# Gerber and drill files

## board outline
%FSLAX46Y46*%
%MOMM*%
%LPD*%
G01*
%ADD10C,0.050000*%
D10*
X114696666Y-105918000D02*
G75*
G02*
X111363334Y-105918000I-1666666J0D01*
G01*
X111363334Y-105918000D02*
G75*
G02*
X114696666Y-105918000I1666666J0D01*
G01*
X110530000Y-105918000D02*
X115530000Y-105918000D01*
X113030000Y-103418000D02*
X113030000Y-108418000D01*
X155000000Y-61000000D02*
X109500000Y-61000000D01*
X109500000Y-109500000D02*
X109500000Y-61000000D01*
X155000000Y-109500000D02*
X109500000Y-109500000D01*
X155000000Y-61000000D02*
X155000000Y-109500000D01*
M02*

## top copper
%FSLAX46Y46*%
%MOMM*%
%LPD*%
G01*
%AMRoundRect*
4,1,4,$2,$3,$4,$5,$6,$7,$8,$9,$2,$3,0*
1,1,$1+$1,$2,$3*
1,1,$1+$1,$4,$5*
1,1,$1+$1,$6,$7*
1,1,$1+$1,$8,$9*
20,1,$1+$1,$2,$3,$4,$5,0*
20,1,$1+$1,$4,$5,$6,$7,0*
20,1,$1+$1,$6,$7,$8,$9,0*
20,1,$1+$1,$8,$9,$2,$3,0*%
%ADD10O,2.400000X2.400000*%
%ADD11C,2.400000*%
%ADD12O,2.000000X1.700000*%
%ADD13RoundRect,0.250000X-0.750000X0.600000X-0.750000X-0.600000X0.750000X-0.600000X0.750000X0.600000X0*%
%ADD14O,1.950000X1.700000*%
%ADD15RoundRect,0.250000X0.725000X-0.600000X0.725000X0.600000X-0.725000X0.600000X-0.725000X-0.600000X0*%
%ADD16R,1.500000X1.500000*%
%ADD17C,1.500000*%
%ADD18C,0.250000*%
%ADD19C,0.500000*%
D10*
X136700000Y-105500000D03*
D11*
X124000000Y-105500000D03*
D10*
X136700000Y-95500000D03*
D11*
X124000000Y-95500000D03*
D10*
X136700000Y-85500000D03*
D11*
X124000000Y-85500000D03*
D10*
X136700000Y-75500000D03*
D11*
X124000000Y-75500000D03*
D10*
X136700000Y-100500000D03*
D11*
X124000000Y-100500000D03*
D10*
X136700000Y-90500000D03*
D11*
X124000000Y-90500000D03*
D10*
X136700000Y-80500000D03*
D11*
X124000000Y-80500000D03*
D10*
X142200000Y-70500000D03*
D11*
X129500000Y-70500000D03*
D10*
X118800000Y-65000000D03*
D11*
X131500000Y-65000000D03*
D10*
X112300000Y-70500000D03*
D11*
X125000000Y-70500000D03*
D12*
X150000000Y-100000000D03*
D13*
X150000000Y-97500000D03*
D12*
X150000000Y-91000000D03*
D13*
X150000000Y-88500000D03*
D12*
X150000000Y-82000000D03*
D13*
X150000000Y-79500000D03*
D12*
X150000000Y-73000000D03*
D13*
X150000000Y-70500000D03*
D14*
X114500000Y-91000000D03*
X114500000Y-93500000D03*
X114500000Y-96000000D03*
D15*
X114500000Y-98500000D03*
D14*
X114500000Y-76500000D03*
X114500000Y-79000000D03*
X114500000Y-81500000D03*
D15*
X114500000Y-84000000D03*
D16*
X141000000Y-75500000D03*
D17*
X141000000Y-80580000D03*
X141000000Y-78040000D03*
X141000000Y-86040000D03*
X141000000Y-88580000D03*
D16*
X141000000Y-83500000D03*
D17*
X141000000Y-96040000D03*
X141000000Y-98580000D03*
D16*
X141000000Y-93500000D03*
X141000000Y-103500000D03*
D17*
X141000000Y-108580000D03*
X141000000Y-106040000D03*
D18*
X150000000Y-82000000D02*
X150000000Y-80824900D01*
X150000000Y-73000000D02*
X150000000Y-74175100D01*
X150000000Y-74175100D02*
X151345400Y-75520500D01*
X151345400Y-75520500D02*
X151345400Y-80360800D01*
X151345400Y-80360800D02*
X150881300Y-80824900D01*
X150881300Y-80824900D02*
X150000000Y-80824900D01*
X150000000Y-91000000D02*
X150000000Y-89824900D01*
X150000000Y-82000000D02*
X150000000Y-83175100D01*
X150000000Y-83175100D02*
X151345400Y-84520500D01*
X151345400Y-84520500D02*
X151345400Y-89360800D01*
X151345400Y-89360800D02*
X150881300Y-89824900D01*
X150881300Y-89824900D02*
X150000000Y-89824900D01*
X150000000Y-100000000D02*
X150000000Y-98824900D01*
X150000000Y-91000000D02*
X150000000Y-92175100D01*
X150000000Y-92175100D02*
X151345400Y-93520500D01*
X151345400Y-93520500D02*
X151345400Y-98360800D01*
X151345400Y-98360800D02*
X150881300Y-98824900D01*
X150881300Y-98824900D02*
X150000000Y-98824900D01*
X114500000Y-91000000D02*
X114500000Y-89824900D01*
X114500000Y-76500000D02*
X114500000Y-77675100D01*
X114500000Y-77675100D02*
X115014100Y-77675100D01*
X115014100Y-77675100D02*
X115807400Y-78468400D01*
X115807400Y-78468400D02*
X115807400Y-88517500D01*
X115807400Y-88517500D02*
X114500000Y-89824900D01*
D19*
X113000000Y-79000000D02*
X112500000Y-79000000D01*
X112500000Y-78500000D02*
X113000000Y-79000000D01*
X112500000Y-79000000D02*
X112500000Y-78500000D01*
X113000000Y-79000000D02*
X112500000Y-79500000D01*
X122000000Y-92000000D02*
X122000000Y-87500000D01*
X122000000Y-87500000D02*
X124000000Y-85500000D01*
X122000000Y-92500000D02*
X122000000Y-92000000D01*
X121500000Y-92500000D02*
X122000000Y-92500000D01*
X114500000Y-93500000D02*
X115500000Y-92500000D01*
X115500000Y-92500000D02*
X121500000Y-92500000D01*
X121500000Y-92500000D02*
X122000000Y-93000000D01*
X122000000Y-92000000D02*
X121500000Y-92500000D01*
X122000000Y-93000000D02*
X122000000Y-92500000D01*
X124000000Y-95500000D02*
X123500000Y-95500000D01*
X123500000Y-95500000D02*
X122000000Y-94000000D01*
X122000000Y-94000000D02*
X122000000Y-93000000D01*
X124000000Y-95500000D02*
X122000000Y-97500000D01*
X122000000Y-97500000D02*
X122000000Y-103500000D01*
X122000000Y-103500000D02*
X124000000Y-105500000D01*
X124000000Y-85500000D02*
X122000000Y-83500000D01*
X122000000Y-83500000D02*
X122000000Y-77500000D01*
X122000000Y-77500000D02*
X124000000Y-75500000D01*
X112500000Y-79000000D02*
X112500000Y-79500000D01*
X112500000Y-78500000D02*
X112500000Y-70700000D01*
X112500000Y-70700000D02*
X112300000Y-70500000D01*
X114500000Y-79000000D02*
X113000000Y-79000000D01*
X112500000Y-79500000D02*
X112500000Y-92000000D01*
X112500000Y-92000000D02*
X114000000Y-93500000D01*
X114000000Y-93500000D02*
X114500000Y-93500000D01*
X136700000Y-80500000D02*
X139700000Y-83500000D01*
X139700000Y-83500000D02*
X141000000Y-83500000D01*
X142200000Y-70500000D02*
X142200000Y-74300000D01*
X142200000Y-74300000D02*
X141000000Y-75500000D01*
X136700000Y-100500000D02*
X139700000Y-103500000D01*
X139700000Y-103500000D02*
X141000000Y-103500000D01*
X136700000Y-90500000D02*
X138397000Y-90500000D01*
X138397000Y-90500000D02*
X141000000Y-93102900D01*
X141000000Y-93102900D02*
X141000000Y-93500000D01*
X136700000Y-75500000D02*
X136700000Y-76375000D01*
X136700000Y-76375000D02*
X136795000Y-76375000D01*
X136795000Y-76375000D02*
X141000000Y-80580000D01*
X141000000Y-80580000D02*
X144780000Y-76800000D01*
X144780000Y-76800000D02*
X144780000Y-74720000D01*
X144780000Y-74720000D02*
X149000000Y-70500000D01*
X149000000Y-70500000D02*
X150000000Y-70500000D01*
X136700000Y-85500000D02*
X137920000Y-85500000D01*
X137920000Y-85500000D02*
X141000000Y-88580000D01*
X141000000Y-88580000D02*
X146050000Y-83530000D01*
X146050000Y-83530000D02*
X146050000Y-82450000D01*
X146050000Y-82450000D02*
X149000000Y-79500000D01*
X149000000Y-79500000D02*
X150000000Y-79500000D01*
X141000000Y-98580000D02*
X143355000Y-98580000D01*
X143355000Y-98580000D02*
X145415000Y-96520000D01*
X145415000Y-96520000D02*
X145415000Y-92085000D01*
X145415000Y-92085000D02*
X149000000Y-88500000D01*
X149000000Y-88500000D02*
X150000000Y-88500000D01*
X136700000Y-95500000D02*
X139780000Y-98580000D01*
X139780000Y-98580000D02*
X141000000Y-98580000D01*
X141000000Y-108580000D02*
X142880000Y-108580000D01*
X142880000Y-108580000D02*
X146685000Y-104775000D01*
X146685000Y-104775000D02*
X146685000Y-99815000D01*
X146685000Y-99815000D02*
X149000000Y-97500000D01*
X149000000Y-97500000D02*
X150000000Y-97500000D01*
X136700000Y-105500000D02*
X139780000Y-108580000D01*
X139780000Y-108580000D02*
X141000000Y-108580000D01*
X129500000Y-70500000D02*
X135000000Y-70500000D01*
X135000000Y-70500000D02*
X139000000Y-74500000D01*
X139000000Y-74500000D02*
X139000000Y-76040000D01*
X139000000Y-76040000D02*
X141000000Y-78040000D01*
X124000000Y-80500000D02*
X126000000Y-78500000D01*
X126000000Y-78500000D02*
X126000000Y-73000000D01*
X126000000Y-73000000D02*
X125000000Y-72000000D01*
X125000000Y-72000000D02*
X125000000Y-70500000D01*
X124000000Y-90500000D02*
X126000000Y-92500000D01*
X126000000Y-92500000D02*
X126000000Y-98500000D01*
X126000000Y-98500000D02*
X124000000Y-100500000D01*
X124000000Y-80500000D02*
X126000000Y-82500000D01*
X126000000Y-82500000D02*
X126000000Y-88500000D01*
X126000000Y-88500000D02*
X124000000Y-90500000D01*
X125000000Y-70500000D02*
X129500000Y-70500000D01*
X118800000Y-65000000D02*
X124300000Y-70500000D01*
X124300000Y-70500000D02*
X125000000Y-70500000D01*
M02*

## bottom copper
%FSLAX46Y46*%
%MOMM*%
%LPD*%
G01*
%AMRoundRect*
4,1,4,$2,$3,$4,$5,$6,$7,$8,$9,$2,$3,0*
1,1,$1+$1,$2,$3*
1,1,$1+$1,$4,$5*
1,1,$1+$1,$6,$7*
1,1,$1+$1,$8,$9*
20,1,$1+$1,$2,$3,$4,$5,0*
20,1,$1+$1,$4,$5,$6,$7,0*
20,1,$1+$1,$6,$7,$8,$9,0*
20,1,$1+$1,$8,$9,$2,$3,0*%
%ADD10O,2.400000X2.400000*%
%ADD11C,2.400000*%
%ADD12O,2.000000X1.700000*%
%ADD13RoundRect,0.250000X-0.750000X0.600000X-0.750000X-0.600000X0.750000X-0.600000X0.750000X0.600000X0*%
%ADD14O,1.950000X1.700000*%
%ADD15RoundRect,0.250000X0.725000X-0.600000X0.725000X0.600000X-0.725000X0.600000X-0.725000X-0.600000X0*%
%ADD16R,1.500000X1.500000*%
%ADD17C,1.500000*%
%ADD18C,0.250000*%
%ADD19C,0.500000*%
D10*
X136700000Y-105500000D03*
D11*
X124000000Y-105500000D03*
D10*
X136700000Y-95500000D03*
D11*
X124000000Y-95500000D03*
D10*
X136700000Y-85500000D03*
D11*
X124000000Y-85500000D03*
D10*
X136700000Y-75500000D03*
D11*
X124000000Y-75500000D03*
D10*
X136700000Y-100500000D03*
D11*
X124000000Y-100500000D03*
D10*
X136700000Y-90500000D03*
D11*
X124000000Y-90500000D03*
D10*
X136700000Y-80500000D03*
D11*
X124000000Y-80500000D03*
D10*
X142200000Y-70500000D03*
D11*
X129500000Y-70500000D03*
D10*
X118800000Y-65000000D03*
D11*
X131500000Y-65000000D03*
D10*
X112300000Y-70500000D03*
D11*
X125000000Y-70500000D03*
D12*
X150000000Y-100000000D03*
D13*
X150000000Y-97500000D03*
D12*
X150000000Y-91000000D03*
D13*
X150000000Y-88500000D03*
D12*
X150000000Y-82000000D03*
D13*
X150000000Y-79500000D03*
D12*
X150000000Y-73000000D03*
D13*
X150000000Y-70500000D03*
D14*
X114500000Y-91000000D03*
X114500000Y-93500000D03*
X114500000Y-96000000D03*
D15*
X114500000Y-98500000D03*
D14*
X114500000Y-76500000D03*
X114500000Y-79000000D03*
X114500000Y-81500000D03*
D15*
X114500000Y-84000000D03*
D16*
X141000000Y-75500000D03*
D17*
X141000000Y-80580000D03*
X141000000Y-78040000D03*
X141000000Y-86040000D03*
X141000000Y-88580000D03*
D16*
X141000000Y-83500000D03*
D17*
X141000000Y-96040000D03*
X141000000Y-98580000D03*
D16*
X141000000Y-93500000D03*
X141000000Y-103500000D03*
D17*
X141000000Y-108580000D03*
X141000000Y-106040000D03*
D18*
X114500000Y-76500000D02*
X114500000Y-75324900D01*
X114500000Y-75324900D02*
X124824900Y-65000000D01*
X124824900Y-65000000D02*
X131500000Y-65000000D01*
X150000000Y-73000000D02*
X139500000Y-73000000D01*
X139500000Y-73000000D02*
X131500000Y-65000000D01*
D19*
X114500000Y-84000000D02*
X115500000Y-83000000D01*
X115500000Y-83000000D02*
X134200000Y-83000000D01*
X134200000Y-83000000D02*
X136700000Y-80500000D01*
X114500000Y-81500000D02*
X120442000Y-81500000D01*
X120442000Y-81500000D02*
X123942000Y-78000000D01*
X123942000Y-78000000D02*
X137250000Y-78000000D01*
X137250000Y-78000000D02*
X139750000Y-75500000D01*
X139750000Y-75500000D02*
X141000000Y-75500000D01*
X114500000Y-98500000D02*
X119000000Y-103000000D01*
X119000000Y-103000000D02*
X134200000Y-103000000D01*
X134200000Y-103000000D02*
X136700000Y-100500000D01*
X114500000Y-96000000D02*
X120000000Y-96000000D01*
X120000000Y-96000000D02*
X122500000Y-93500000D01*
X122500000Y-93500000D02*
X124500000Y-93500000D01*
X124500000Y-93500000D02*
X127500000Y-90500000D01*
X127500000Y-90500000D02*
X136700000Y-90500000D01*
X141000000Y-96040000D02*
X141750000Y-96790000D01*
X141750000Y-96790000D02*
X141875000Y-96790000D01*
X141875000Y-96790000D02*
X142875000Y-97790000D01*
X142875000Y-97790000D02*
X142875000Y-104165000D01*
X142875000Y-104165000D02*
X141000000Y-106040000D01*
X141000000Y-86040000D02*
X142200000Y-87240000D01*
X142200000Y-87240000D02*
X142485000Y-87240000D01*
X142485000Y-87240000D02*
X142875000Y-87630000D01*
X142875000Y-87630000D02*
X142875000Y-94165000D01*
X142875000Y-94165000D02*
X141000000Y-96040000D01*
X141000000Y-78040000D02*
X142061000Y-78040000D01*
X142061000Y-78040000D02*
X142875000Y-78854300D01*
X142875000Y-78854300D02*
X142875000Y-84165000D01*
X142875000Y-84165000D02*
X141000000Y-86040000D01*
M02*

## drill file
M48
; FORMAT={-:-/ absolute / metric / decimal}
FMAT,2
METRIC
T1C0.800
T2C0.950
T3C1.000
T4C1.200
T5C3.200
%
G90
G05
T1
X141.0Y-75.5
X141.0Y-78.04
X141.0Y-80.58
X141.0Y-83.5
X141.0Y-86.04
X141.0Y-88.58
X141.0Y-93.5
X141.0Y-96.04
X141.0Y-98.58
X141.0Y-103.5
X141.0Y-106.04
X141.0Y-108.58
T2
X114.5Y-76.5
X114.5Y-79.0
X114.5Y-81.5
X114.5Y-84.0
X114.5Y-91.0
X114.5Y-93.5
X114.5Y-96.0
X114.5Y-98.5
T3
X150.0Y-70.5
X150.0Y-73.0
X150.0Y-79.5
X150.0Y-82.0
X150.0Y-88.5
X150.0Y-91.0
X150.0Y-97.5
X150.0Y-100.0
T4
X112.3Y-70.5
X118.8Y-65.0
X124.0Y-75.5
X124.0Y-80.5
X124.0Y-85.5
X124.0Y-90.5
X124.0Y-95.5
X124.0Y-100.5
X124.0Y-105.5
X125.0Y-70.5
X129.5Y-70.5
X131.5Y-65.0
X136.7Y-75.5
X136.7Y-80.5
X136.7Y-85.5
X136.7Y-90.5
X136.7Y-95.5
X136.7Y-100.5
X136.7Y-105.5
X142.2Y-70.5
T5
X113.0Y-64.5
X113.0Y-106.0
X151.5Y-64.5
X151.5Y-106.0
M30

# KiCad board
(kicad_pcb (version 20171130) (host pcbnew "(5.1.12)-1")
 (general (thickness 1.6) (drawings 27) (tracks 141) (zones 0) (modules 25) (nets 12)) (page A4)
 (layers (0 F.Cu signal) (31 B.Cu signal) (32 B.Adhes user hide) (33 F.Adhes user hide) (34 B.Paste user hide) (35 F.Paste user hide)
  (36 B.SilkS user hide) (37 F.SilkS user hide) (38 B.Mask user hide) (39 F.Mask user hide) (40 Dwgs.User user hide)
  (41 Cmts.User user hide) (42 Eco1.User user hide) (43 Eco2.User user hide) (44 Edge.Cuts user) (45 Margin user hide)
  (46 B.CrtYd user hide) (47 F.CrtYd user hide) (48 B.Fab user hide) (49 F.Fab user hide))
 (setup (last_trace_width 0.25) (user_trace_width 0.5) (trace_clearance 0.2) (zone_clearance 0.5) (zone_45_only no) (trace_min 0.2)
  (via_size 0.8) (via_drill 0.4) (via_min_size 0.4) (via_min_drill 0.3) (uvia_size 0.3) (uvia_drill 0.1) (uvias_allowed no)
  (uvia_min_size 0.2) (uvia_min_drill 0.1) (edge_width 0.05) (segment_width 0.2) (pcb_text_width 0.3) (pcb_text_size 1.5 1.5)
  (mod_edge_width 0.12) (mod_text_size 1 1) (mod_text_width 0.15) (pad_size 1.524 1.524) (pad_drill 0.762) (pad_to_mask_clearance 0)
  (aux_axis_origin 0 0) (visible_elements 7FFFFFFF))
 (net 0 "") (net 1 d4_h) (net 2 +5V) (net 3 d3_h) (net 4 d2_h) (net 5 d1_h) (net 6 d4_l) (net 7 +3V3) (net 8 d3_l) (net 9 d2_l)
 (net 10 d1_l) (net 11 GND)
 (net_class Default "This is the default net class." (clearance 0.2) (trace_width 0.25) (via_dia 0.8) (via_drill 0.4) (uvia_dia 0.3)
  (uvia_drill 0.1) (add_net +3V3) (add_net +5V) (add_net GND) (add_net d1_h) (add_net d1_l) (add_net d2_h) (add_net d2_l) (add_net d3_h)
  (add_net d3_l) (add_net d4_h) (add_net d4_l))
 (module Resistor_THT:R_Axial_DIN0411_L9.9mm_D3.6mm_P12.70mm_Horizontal (layer F.Cu) (at 124 105.5)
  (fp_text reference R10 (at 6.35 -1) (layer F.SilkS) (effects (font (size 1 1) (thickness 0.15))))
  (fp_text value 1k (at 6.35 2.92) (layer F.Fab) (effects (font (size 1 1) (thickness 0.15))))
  (pad 2 thru_hole oval (at 12.7 0) (size 2.4 2.4) (drill 1.2) (layers *.Cu *.Mask) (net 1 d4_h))
  (pad 1 thru_hole circle (at 0 0) (size 2.4 2.4) (drill 1.2) (layers *.Cu *.Mask) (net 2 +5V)))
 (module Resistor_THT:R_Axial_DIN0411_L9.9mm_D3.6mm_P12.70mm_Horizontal (layer F.Cu) (at 124 95.5)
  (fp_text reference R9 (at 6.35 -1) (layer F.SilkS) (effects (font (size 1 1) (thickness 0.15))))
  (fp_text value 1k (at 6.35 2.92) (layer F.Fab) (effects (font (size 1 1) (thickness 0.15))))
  (pad 2 thru_hole oval (at 12.7 0) (size 2.4 2.4) (drill 1.2) (layers *.Cu *.Mask) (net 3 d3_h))
  (pad 1 thru_hole circle (at 0 0) (size 2.4 2.4) (drill 1.2) (layers *.Cu *.Mask) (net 2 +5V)))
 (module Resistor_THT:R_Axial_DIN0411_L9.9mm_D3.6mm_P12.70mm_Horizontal (layer F.Cu) (at 124 85.5)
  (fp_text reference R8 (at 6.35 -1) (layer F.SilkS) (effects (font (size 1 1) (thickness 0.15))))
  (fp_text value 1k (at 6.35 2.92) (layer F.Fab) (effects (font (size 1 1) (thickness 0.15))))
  (pad 2 thru_hole oval (at 12.7 0) (size 2.4 2.4) (drill 1.2) (layers *.Cu *.Mask) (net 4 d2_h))
  (pad 1 thru_hole circle (at 0 0) (size 2.4 2.4) (drill 1.2) (layers *.Cu *.Mask) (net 2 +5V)))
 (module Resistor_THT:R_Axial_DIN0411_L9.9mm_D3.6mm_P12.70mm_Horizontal (layer F.Cu) (at 124 75.5)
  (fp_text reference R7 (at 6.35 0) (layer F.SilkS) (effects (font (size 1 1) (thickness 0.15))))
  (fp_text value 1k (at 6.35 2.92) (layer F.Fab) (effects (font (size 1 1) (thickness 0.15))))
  (pad 2 thru_hole oval (at 12.7 0) (size 2.4 2.4) (drill 1.2) (layers *.Cu *.Mask) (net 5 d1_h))
  (pad 1 thru_hole circle (at 0 0) (size 2.4 2.4) (drill 1.2) (layers *.Cu *.Mask) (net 2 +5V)))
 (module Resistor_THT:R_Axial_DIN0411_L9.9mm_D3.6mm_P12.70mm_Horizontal (layer F.Cu) (at 124 100.5)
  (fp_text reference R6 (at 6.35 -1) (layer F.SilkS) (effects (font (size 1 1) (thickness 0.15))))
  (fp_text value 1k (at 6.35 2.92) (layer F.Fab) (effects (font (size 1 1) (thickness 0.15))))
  (pad 2 thru_hole oval (at 12.7 0) (size 2.4 2.4) (drill 1.2) (layers *.Cu *.Mask) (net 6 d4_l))
  (pad 1 thru_hole circle (at 0 0) (size 2.4 2.4) (drill 1.2) (layers *.Cu *.Mask) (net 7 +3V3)))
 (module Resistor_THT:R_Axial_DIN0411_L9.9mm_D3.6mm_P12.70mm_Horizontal (layer F.Cu) (at 124 90.5)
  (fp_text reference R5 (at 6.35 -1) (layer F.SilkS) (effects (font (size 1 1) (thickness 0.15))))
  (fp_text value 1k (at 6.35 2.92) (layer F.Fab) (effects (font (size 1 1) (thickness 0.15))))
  (pad 2 thru_hole oval (at 12.7 0) (size 2.4 2.4) (drill 1.2) (layers *.Cu *.Mask) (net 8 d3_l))
  (pad 1 thru_hole circle (at 0 0) (size 2.4 2.4) (drill 1.2) (layers *.Cu *.Mask) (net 7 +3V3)))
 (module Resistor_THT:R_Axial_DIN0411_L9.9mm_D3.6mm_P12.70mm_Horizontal (layer F.Cu) (at 124 80.5)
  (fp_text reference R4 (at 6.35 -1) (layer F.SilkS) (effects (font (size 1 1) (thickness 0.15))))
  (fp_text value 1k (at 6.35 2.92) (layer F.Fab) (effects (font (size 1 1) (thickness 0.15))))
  (pad 2 thru_hole oval (at 12.7 0) (size 2.4 2.4) (drill 1.2) (layers *.Cu *.Mask) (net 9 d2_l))
  (pad 1 thru_hole circle (at 0 0) (size 2.4 2.4) (drill 1.2) (layers *.Cu *.Mask) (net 7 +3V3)))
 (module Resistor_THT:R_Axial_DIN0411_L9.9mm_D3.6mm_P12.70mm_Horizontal (layer F.Cu) (at 129.5 70.5)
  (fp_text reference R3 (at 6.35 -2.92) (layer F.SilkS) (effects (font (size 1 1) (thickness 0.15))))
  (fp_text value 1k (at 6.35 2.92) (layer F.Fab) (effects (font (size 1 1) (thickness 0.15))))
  (pad 2 thru_hole oval (at 12.7 0) (size 2.4 2.4) (drill 1.2) (layers *.Cu *.Mask) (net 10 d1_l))
  (pad 1 thru_hole circle (at 0 0) (size 2.4 2.4) (drill 1.2) (layers *.Cu *.Mask) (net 7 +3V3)))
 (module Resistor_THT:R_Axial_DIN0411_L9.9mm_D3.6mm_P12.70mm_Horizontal (layer F.Cu) (at 131.5 65 180)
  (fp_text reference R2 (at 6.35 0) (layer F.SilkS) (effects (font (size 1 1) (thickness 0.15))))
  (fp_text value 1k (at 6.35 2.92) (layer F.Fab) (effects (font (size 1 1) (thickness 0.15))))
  (pad 2 thru_hole oval (at 12.7 0 180) (size 2.4 2.4) (drill 1.2) (layers *.Cu *.Mask) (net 7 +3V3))
  (pad 1 thru_hole circle (at 0 0 180) (size 2.4 2.4) (drill 1.2) (layers *.Cu *.Mask) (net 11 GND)))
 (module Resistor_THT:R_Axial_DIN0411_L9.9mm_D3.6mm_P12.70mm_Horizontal (layer F.Cu) (at 125 70.5 180)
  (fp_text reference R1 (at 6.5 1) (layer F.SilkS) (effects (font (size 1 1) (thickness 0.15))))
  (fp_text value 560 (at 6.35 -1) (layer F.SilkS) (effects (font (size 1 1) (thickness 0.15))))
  (pad 2 thru_hole oval (at 12.7 0 180) (size 2.4 2.4) (drill 1.2) (layers *.Cu *.Mask) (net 2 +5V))
  (pad 1 thru_hole circle (at 0 0 180) (size 2.4 2.4) (drill 1.2) (layers *.Cu *.Mask) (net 7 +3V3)))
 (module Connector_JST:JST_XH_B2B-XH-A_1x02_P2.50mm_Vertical (layer F.Cu) (at 150 97.5 270)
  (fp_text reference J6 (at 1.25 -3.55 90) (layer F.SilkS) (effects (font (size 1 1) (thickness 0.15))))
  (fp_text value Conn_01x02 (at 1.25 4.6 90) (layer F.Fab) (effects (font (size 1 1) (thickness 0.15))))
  (pad 2 thru_hole oval (at 2.5 0 270) (size 1.7 2) (drill 1) (layers *.Cu *.Mask) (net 11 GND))
  (pad 1 thru_hole roundrect (at 0 0 270) (size 1.7 2) (drill 1) (layers *.Cu *.Mask) (roundrect_rratio 0.1470588235294118) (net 1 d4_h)))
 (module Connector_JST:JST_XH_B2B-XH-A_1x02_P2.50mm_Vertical (layer F.Cu) (at 150 88.5 270)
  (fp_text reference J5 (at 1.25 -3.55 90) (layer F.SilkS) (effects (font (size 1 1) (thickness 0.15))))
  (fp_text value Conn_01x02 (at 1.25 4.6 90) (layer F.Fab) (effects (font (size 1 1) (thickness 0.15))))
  (pad 2 thru_hole oval (at 2.5 0 270) (size 1.7 2) (drill 1) (layers *.Cu *.Mask) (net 11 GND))
  (pad 1 thru_hole roundrect (at 0 0 270) (size 1.7 2) (drill 1) (layers *.Cu *.Mask) (roundrect_rratio 0.1470588235294118) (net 3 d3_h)))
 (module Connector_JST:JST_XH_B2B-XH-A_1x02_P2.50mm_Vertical (layer F.Cu) (at 150 79.5 270)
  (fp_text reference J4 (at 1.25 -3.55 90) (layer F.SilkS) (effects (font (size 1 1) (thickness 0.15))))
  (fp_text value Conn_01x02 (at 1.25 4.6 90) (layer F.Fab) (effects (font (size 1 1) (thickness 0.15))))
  (pad 2 thru_hole oval (at 2.5 0 270) (size 1.7 2) (drill 1) (layers *.Cu *.Mask) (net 11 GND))
  (pad 1 thru_hole roundrect (at 0 0 270) (size 1.7 2) (drill 1) (layers *.Cu *.Mask) (roundrect_rratio 0.1470588235294118) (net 4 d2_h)))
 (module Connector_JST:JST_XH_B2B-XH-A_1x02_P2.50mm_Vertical (layer F.Cu) (at 150 70.5 270)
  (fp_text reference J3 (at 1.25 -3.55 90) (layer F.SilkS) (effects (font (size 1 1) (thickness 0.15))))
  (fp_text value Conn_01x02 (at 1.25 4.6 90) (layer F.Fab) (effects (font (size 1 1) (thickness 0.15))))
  (pad 2 thru_hole oval (at 2.5 0 270) (size 1.7 2) (drill 1) (layers *.Cu *.Mask) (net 11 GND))
  (pad 1 thru_hole roundrect (at 0 0 270) (size 1.7 2) (drill 1) (layers *.Cu *.Mask) (roundrect_rratio 0.1470588235294118) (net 5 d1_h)))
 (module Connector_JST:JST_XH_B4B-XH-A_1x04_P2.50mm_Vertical (layer F.Cu) (at 114.5 98.5 90)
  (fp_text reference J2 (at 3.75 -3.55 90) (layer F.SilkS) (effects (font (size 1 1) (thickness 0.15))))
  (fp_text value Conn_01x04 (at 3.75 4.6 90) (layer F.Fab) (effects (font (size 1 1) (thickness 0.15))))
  (pad 4 thru_hole oval (at 7.5 0 90) (size 1.7 1.95) (drill 0.95) (layers *.Cu *.Mask) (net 11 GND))
  (pad 3 thru_hole oval (at 5 0 90) (size 1.7 1.95) (drill 0.95) (layers *.Cu *.Mask) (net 2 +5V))
  (pad 2 thru_hole oval (at 2.5 0 90) (size 1.7 1.95) (drill 0.95) (layers *.Cu *.Mask) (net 8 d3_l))
  (pad 1 thru_hole roundrect (at 0 0 90) (size 1.7 1.95) (drill 0.95) (layers *.Cu *.Mask) (roundrect_rratio 0.1470588235294118)
   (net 6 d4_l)))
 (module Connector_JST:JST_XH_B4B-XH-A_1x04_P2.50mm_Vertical (layer F.Cu) (at 114.5 84 90)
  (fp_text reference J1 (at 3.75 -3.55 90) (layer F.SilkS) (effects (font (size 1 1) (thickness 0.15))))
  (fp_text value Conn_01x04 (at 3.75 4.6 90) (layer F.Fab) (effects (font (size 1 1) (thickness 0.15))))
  (pad 4 thru_hole oval (at 7.5 0 90) (size 1.7 1.95) (drill 0.95) (layers *.Cu *.Mask) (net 11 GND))
  (pad 3 thru_hole oval (at 5 0 90) (size 1.7 1.95) (drill 0.95) (layers *.Cu *.Mask) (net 2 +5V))
  (pad 2 thru_hole oval (at 2.5 0 90) (size 1.7 1.95) (drill 0.95) (layers *.Cu *.Mask) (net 10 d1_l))
  (pad 1 thru_hole roundrect (at 0 0 90) (size 1.7 1.95) (drill 0.95) (layers *.Cu *.Mask) (roundrect_rratio 0.1470588235294118)
   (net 9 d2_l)))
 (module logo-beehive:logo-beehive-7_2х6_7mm (layer F.Cu) (at 140 65)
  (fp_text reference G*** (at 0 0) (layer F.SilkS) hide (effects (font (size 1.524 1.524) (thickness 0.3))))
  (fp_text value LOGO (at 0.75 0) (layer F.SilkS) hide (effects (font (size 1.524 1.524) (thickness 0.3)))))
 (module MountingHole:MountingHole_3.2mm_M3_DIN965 (layer F.Cu) (at 113 106)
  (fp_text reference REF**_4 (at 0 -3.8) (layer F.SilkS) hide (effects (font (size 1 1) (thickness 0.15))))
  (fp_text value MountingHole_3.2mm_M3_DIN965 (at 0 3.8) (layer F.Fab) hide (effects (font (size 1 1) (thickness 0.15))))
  (pad 1 np_thru_hole circle (at 0 0) (size 3.2 3.2) (drill 3.2) (layers *.Cu *.Mask)))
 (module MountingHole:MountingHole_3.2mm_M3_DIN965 (layer F.Cu) (at 151.5 64.5)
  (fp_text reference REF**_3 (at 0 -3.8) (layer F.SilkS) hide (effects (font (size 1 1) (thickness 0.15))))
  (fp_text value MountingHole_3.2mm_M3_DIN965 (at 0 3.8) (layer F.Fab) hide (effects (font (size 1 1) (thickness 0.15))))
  (pad 1 np_thru_hole circle (at 0 0) (size 3.2 3.2) (drill 3.2) (layers *.Cu *.Mask)))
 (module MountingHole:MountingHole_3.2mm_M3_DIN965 (layer F.Cu) (at 113 64.5)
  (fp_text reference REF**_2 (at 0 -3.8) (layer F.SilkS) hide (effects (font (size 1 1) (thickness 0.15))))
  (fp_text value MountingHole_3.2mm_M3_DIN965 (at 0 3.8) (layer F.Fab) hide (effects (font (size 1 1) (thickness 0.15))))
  (pad 1 np_thru_hole circle (at 0 0) (size 3.2 3.2) (drill 3.2) (layers *.Cu *.Mask)))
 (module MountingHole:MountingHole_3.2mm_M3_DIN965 (layer F.Cu) (at 151.5 106)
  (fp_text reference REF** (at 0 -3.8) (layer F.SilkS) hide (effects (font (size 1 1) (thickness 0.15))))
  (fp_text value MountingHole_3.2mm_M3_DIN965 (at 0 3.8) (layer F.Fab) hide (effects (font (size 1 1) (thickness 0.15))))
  (pad 1 np_thru_hole circle (at 0 0) (size 3.2 3.2) (drill 3.2) (layers *.Cu *.Mask)))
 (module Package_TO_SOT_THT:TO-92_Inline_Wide (layer F.Cu) (at 141 75.5 270)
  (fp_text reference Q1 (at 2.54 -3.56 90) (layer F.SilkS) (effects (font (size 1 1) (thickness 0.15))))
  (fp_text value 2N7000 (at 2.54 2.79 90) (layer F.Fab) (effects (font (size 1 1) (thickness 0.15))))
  (pad 1 thru_hole rect (at 0 0) (size 1.5 1.5) (drill 0.8) (layers *.Cu *.Mask) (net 10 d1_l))
  (pad 3 thru_hole circle (at 5.08 0) (size 1.5 1.5) (drill 0.8) (layers *.Cu *.Mask) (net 5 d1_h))
  (pad 2 thru_hole circle (at 2.54 0) (size 1.5 1.5) (drill 0.8) (layers *.Cu *.Mask) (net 7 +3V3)))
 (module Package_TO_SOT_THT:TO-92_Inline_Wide (layer F.Cu) (at 141 83.5 270)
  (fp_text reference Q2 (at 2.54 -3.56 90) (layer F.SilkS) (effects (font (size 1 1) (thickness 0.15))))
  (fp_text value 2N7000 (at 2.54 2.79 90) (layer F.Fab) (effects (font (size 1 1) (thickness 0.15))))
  (pad 2 thru_hole circle (at 2.54 0) (size 1.5 1.5) (drill 0.8) (layers *.Cu *.Mask) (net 7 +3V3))
  (pad 3 thru_hole circle (at 5.08 0) (size 1.5 1.5) (drill 0.8) (layers *.Cu *.Mask) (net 4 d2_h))
  (pad 1 thru_hole rect (at 0 0) (size 1.5 1.5) (drill 0.8) (layers *.Cu *.Mask) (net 9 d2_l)))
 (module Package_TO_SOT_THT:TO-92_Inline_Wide (layer F.Cu) (at 141 93.5 270)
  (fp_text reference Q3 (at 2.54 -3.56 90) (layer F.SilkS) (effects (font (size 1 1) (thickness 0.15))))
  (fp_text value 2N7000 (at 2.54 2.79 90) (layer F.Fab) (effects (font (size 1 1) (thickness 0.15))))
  (pad 2 thru_hole circle (at 2.54 0) (size 1.5 1.5) (drill 0.8) (layers *.Cu *.Mask) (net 7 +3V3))
  (pad 3 thru_hole circle (at 5.08 0) (size 1.5 1.5) (drill 0.8) (layers *.Cu *.Mask) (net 3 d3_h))
  (pad 1 thru_hole rect (at 0 0) (size 1.5 1.5) (drill 0.8) (layers *.Cu *.Mask) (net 8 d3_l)))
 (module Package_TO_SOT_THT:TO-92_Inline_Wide (layer F.Cu) (at 141 103.5 270)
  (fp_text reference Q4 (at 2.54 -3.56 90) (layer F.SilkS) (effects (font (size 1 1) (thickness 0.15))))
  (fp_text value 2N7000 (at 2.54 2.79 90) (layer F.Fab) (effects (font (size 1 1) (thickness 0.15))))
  (pad 1 thru_hole rect (at 0 0) (size 1.5 1.5) (drill 0.8) (layers *.Cu *.Mask) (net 6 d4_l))
  (pad 3 thru_hole circle (at 5.08 0) (size 1.5 1.5) (drill 0.8) (layers *.Cu *.Mask) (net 1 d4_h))
  (pad 2 thru_hole circle (at 2.54 0) (size 1.5 1.5) (drill 0.8) (layers *.Cu *.Mask) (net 7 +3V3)))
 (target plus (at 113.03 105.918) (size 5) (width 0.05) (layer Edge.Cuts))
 (gr_line (start 155 61) (end 109.5 61) (layer Edge.Cuts) (width 0.05))
 (gr_line (start 109.5 109.5) (end 109.5 61) (layer Edge.Cuts) (width 0.05))
 (gr_line (start 155 109.5) (end 109.5 109.5) (layer Edge.Cuts) (width 0.05))
 (gr_line (start 155 61) (end 155 109.5) (layer Edge.Cuts) (width 0.05))
 (segment (start 150 82) (end 150 80.8249) (width 0.25) (layer F.Cu) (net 11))
 (segment (start 150 73) (end 150 74.1751) (width 0.25) (layer F.Cu) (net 11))
 (segment (start 150 74.1751) (end 151.3454 75.5205) (width 0.25) (layer F.Cu) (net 11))
 (segment (start 151.3454 75.5205) (end 151.3454 80.3608) (width 0.25) (layer F.Cu) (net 11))
 (segment (start 151.3454 80.3608) (end 150.8813 80.8249) (width 0.25) (layer F.Cu) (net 11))
 (segment (start 150.8813 80.8249) (end 150 80.8249) (width 0.25) (layer F.Cu) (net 11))
 (segment (start 114.5 76.5) (end 114.5 75.3249) (width 0.25) (layer B.Cu) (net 11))
 (segment (start 114.5 75.3249) (end 124.8249 65) (width 0.25) (layer B.Cu) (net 11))
 (segment (start 124.8249 65) (end 131.5 65) (width 0.25) (layer B.Cu) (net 11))
 (segment (start 150 91) (end 150 89.8249) (width 0.25) (layer F.Cu) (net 11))
 (segment (start 150 82) (end 150 83.1751) (width 0.25) (layer F.Cu) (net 11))
 (segment (start 150 83.1751) (end 151.3454 84.5205) (width 0.25) (layer F.Cu) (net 11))
 (segment (start 151.3454 84.5205) (end 151.3454 89.3608) (width 0.25) (layer F.Cu) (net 11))
 (segment (start 151.3454 89.3608) (end 150.8813 89.8249) (width 0.25) (layer F.Cu) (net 11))
 (segment (start 150.8813 89.8249) (end 150 89.8249) (width 0.25) (layer F.Cu) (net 11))
 (segment (start 150 73) (end 139.5 73) (width 0.25) (layer B.Cu) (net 11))
 (segment (start 139.5 73) (end 131.5 65) (width 0.25) (layer B.Cu) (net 11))
 (segment (start 150 100) (end 150 98.8249) (width 0.25) (layer F.Cu) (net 11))
 (segment (start 150 91) (end 150 92.1751) (width 0.25) (layer F.Cu) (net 11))
 (segment (start 150 92.1751) (end 151.3454 93.5205) (width 0.25) (layer F.Cu) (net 11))
 (segment (start 151.3454 93.5205) (end 151.3454 98.3608) (width 0.25) (layer F.Cu) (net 11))
 (segment (start 151.3454 98.3608) (end 150.8813 98.8249) (width 0.25) (layer F.Cu) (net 11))
 (segment (start 150.8813 98.8249) (end 150 98.8249) (width 0.25) (layer F.Cu) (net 11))
 (segment (start 114.5 91) (end 114.5 89.8249) (width 0.25) (layer F.Cu) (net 11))
 (segment (start 114.5 76.5) (end 114.5 77.6751) (width 0.25) (layer F.Cu) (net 11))
 (segment (start 114.5 77.6751) (end 115.0141 77.6751) (width 0.25) (layer F.Cu) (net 11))
 (segment (start 115.0141 77.6751) (end 115.8074 78.4684) (width 0.25) (layer F.Cu) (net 11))
 (segment (start 115.8074 78.4684) (end 115.8074 88.5175) (width 0.25) (layer F.Cu) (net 11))
 (segment (start 115.8074 88.5175) (end 114.5 89.8249) (width 0.25) (layer F.Cu) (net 11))
 (segment (start 113 79) (end 112.5 79) (width 0.5) (layer F.Cu) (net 2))
 (segment (start 112.5 78.5) (end 113 79) (width 0.5) (layer F.Cu) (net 2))
 (segment (start 112.5 79) (end 112.5 78.5) (width 0.5) (layer F.Cu) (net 2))
 (segment (start 113 79) (end 112.5 79.5) (width 0.5) (layer F.Cu) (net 2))
 (segment (start 122 92) (end 122 87.5) (width 0.5) (layer F.Cu) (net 2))
 (segment (start 122 87.5) (end 124 85.5) (width 0.5) (layer F.Cu) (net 2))
 (segment (start 122 92.5) (end 122 92) (width 0.5) (layer F.Cu) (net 2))
 (segment (start 121.5 92.5) (end 122 92.5) (width 0.5) (layer F.Cu) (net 2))
 (segment (start 114.5 93.5) (end 115.5 92.5) (width 0.5) (layer F.Cu) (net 2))
 (segment (start 115.5 92.5) (end 121.5 92.5) (width 0.5) (layer F.Cu) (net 2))
 (segment (start 121.5 92.5) (end 122 93) (width 0.5) (layer F.Cu) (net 2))
 (segment (start 122 92) (end 121.5 92.5) (width 0.5) (layer F.Cu) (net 2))
 (segment (start 122 93) (end 122 92.5) (width 0.5) (layer F.Cu) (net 2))
 (segment (start 124 95.5) (end 123.5 95.5) (width 0.5) (layer F.Cu) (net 2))
 (segment (start 123.5 95.5) (end 122 94) (width 0.5) (layer F.Cu) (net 2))
 (segment (start 122 94) (end 122 93) (width 0.5) (layer F.Cu) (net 2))
 (segment (start 124 95.5) (end 122 97.5) (width 0.5) (layer F.Cu) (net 2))
 (segment (start 122 97.5) (end 122 103.5) (width 0.5) (layer F.Cu) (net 2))
 (segment (start 122 103.5) (end 124 105.5) (width 0.5) (layer F.Cu) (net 2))
 (segment (start 124 85.5) (end 122 83.5) (width 0.5) (layer F.Cu) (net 2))
 (segment (start 122 83.5) (end 122 77.5) (width 0.5) (layer F.Cu) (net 2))
 (segment (start 122 77.5) (end 124 75.5) (width 0.5) (layer F.Cu) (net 2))
 (segment (start 112.5 79) (end 112.5 79.5) (width 0.5) (layer F.Cu) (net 2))
 (segment (start 112.5 78.5) (end 112.5 70.7) (width 0.5) (layer F.Cu) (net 2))
 (segment (start 112.5 70.7) (end 112.3 70.5) (width 0.5) (layer F.Cu) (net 2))
 (segment (start 114.5 79) (end 113 79) (width 0.5) (layer F.Cu) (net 2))
 (segment (start 112.5 79.5) (end 112.5 92) (width 0.5) (layer F.Cu) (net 2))
 (segment (start 112.5 92) (end 114 93.5) (width 0.5) (layer F.Cu) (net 2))
 (segment (start 114 93.5) (end 114.5 93.5) (width 0.5) (layer F.Cu) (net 2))
 (segment (start 136.7 80.5) (end 139.7 83.5) (width 0.5) (layer F.Cu) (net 9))
 (segment (start 139.7 83.5) (end 141 83.5) (width 0.5) (layer F.Cu) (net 9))
 (segment (start 114.5 84) (end 115.5 83) (width 0.5) (layer B.Cu) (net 9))
 (segment (start 115.5 83) (end 134.2 83) (width 0.5) (layer B.Cu) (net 9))
 (segment (start 134.2 83) (end 136.7 80.5) (width 0.5) (layer B.Cu) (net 9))
 (segment (start 114.5 81.5) (end 120.442 81.5) (width 0.5) (layer B.Cu) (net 10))
 (segment (start 120.442 81.5) (end 123.942 78) (width 0.5) (layer B.Cu) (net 10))
 (segment (start 123.942 78) (end 137.25 78) (width 0.5) (layer B.Cu) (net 10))
 (segment (start 137.25 78) (end 139.75 75.5) (width 0.5) (layer B.Cu) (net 10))
 (segment (start 139.75 75.5) (end 141 75.5) (width 0.5) (layer B.Cu) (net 10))
 (segment (start 142.2 70.5) (end 142.2 74.3) (width 0.5) (layer F.Cu) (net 10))
 (segment (start 142.2 74.3) (end 141 75.5) (width 0.5) (layer F.Cu) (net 10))
 (segment (start 114.5 98.5) (end 119 103) (width 0.5) (layer B.Cu) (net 6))
 (segment (start 119 103) (end 134.2 103) (width 0.5) (layer B.Cu) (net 6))
 (segment (start 134.2 103) (end 136.7 100.5) (width 0.5) (layer B.Cu) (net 6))
 (segment (start 136.7 100.5) (end 139.7 103.5) (width 0.5) (layer F.Cu) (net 6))
 (segment (start 139.7 103.5) (end 141 103.5) (width 0.5) (layer F.Cu) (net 6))
 (segment (start 114.5 96) (end 120 96) (width 0.5) (layer B.Cu) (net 8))
 (segment (start 120 96) (end 122.5 93.5) (width 0.5) (layer B.Cu) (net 8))
 (segment (start 122.5 93.5) (end 124.5 93.5) (width 0.5) (layer B.Cu) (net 8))
 (segment (start 124.5 93.5) (end 127.5 90.5) (width 0.5) (layer B.Cu) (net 8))
 (segment (start 127.5 90.5) (end 136.7 90.5) (width 0.5) (layer B.Cu) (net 8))
 (segment (start 136.7 90.5) (end 138.397 90.5) (width 0.5) (layer F.Cu) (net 8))
 (segment (start 138.397 90.5) (end 141 93.1029) (width 0.5) (layer F.Cu) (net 8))
 (segment (start 141 93.1029) (end 141 93.5) (width 0.5) (layer F.Cu) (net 8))
 (segment (start 136.7 75.5) (end 136.7 76.375) (width 0.5) (layer F.Cu) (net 5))
 (segment (start 136.7 76.375) (end 136.795 76.375) (width 0.5) (layer F.Cu) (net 5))
 (segment (start 136.795 76.375) (end 141 80.58) (width 0.5) (layer F.Cu) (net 5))
 (segment (start 141 80.58) (end 144.78 76.8) (width 0.5) (layer F.Cu) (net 5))
 (segment (start 144.78 76.8) (end 144.78 74.72) (width 0.5) (layer F.Cu) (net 5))
 (segment (start 144.78 74.72) (end 149 70.5) (width 0.5) (layer F.Cu) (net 5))
 (segment (start 149 70.5) (end 150 70.5) (width 0.5) (layer F.Cu) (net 5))
 (segment (start 136.7 85.5) (end 137.92 85.5) (width 0.5) (layer F.Cu) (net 4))
 (segment (start 137.92 85.5) (end 141 88.58) (width 0.5) (layer F.Cu) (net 4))
 (segment (start 141 88.58) (end 146.05 83.53) (width 0.5) (layer F.Cu) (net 4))
 (segment (start 146.05 83.53) (end 146.05 82.45) (width 0.5) (layer F.Cu) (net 4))
 (segment (start 146.05 82.45) (end 149 79.5) (width 0.5) (layer F.Cu) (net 4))
 (segment (start 149 79.5) (end 150 79.5) (width 0.5) (layer F.Cu) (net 4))
 (segment (start 141 98.58) (end 143.355 98.58) (width 0.5) (layer F.Cu) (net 3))
 (segment (start 143.355 98.58) (end 145.415 96.52) (width 0.5) (layer F.Cu) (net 3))
 (segment (start 145.415 96.52) (end 145.415 92.085) (width 0.5) (layer F.Cu) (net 3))
 (segment (start 145.415 92.085) (end 149 88.5) (width 0.5) (layer F.Cu) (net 3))
 (segment (start 149 88.5) (end 150 88.5) (width 0.5) (layer F.Cu) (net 3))
 (segment (start 136.7 95.5) (end 139.78 98.58) (width 0.5) (layer F.Cu) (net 3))
 (segment (start 139.78 98.58) (end 141 98.58) (width 0.5) (layer F.Cu) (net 3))
 (segment (start 141 108.58) (end 142.88 108.58) (width 0.5) (layer F.Cu) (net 1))
 (segment (start 142.88 108.58) (end 146.685 104.775) (width 0.5) (layer F.Cu) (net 1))
 (segment (start 146.685 104.775) (end 146.685 99.815) (width 0.5) (layer F.Cu) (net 1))
 (segment (start 146.685 99.815) (end 149 97.5) (width 0.5) (layer F.Cu) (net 1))
 (segment (start 149 97.5) (end 150 97.5) (width 0.5) (layer F.Cu) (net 1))
 (segment (start 136.7 105.5) (end 139.78 108.58) (width 0.5) (layer F.Cu) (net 1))
 (segment (start 139.78 108.58) (end 141 108.58) (width 0.5) (layer F.Cu) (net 1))
 (segment (start 141 96.04) (end 141.75 96.79) (width 0.5) (layer B.Cu) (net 7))
 (segment (start 141.75 96.79) (end 141.875 96.79) (width 0.5) (layer B.Cu) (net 7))
 (segment (start 141.875 96.79) (end 142.875 97.79) (width 0.5) (layer B.Cu) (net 7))
 (segment (start 142.875 97.79) (end 142.875 104.165) (width 0.5) (layer B.Cu) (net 7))
 (segment (start 142.875 104.165) (end 141 106.04) (width 0.5) (layer B.Cu) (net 7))
 (segment (start 141 86.04) (end 142.2 87.24) (width 0.5) (layer B.Cu) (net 7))
 (segment (start 142.2 87.24) (end 142.485 87.24) (width 0.5) (layer B.Cu) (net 7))
 (segment (start 142.485 87.24) (end 142.875 87.63) (width 0.5) (layer B.Cu) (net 7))
 (segment (start 142.875 87.63) (end 142.875 94.165) (width 0.5) (layer B.Cu) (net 7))
 (segment (start 142.875 94.165) (end 141 96.04) (width 0.5) (layer B.Cu) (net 7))
 (segment (start 141 78.04) (end 142.061 78.04) (width 0.5) (layer B.Cu) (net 7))
 (segment (start 142.061 78.04) (end 142.875 78.8543) (width 0.5) (layer B.Cu) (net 7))
 (segment (start 142.875 78.8543) (end 142.875 84.165) (width 0.5) (layer B.Cu) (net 7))
 (segment (start 142.875 84.165) (end 141 86.04) (width 0.5) (layer B.Cu) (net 7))
 (segment (start 129.5 70.5) (end 135 70.5) (width 0.5) (layer F.Cu) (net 7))
 (segment (start 135 70.5) (end 139 74.5) (width 0.5) (layer F.Cu) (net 7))
 (segment (start 139 74.5) (end 139 76.04) (width 0.5) (layer F.Cu) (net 7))
 (segment (start 139 76.04) (end 141 78.04) (width 0.5) (layer F.Cu) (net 7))
 (segment (start 124 80.5) (end 126 78.5) (width 0.5) (layer F.Cu) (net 7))
 (segment (start 126 78.5) (end 126 73) (width 0.5) (layer F.Cu) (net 7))
 (segment (start 126 73) (end 125 72) (width 0.5) (layer F.Cu) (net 7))
 (segment (start 125 72) (end 125 70.5) (width 0.5) (layer F.Cu) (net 7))
 (segment (start 124 90.5) (end 126 92.5) (width 0.5) (layer F.Cu) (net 7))
 (segment (start 126 92.5) (end 126 98.5) (width 0.5) (layer F.Cu) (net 7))
 (segment (start 126 98.5) (end 124 100.5) (width 0.5) (layer F.Cu) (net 7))
 (segment (start 124 80.5) (end 126 82.5) (width 0.5) (layer F.Cu) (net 7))
 (segment (start 126 82.5) (end 126 88.5) (width 0.5) (layer F.Cu) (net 7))
 (segment (start 126 88.5) (end 124 90.5) (width 0.5) (layer F.Cu) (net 7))
 (segment (start 125 70.5) (end 129.5 70.5) (width 0.5) (layer F.Cu) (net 7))
 (segment (start 118.8 65) (end 124.3 70.5) (width 0.5) (layer F.Cu) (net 7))
 (segment (start 124.3 70.5) (end 125 70.5) (width 0.5) (layer F.Cu) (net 7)))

